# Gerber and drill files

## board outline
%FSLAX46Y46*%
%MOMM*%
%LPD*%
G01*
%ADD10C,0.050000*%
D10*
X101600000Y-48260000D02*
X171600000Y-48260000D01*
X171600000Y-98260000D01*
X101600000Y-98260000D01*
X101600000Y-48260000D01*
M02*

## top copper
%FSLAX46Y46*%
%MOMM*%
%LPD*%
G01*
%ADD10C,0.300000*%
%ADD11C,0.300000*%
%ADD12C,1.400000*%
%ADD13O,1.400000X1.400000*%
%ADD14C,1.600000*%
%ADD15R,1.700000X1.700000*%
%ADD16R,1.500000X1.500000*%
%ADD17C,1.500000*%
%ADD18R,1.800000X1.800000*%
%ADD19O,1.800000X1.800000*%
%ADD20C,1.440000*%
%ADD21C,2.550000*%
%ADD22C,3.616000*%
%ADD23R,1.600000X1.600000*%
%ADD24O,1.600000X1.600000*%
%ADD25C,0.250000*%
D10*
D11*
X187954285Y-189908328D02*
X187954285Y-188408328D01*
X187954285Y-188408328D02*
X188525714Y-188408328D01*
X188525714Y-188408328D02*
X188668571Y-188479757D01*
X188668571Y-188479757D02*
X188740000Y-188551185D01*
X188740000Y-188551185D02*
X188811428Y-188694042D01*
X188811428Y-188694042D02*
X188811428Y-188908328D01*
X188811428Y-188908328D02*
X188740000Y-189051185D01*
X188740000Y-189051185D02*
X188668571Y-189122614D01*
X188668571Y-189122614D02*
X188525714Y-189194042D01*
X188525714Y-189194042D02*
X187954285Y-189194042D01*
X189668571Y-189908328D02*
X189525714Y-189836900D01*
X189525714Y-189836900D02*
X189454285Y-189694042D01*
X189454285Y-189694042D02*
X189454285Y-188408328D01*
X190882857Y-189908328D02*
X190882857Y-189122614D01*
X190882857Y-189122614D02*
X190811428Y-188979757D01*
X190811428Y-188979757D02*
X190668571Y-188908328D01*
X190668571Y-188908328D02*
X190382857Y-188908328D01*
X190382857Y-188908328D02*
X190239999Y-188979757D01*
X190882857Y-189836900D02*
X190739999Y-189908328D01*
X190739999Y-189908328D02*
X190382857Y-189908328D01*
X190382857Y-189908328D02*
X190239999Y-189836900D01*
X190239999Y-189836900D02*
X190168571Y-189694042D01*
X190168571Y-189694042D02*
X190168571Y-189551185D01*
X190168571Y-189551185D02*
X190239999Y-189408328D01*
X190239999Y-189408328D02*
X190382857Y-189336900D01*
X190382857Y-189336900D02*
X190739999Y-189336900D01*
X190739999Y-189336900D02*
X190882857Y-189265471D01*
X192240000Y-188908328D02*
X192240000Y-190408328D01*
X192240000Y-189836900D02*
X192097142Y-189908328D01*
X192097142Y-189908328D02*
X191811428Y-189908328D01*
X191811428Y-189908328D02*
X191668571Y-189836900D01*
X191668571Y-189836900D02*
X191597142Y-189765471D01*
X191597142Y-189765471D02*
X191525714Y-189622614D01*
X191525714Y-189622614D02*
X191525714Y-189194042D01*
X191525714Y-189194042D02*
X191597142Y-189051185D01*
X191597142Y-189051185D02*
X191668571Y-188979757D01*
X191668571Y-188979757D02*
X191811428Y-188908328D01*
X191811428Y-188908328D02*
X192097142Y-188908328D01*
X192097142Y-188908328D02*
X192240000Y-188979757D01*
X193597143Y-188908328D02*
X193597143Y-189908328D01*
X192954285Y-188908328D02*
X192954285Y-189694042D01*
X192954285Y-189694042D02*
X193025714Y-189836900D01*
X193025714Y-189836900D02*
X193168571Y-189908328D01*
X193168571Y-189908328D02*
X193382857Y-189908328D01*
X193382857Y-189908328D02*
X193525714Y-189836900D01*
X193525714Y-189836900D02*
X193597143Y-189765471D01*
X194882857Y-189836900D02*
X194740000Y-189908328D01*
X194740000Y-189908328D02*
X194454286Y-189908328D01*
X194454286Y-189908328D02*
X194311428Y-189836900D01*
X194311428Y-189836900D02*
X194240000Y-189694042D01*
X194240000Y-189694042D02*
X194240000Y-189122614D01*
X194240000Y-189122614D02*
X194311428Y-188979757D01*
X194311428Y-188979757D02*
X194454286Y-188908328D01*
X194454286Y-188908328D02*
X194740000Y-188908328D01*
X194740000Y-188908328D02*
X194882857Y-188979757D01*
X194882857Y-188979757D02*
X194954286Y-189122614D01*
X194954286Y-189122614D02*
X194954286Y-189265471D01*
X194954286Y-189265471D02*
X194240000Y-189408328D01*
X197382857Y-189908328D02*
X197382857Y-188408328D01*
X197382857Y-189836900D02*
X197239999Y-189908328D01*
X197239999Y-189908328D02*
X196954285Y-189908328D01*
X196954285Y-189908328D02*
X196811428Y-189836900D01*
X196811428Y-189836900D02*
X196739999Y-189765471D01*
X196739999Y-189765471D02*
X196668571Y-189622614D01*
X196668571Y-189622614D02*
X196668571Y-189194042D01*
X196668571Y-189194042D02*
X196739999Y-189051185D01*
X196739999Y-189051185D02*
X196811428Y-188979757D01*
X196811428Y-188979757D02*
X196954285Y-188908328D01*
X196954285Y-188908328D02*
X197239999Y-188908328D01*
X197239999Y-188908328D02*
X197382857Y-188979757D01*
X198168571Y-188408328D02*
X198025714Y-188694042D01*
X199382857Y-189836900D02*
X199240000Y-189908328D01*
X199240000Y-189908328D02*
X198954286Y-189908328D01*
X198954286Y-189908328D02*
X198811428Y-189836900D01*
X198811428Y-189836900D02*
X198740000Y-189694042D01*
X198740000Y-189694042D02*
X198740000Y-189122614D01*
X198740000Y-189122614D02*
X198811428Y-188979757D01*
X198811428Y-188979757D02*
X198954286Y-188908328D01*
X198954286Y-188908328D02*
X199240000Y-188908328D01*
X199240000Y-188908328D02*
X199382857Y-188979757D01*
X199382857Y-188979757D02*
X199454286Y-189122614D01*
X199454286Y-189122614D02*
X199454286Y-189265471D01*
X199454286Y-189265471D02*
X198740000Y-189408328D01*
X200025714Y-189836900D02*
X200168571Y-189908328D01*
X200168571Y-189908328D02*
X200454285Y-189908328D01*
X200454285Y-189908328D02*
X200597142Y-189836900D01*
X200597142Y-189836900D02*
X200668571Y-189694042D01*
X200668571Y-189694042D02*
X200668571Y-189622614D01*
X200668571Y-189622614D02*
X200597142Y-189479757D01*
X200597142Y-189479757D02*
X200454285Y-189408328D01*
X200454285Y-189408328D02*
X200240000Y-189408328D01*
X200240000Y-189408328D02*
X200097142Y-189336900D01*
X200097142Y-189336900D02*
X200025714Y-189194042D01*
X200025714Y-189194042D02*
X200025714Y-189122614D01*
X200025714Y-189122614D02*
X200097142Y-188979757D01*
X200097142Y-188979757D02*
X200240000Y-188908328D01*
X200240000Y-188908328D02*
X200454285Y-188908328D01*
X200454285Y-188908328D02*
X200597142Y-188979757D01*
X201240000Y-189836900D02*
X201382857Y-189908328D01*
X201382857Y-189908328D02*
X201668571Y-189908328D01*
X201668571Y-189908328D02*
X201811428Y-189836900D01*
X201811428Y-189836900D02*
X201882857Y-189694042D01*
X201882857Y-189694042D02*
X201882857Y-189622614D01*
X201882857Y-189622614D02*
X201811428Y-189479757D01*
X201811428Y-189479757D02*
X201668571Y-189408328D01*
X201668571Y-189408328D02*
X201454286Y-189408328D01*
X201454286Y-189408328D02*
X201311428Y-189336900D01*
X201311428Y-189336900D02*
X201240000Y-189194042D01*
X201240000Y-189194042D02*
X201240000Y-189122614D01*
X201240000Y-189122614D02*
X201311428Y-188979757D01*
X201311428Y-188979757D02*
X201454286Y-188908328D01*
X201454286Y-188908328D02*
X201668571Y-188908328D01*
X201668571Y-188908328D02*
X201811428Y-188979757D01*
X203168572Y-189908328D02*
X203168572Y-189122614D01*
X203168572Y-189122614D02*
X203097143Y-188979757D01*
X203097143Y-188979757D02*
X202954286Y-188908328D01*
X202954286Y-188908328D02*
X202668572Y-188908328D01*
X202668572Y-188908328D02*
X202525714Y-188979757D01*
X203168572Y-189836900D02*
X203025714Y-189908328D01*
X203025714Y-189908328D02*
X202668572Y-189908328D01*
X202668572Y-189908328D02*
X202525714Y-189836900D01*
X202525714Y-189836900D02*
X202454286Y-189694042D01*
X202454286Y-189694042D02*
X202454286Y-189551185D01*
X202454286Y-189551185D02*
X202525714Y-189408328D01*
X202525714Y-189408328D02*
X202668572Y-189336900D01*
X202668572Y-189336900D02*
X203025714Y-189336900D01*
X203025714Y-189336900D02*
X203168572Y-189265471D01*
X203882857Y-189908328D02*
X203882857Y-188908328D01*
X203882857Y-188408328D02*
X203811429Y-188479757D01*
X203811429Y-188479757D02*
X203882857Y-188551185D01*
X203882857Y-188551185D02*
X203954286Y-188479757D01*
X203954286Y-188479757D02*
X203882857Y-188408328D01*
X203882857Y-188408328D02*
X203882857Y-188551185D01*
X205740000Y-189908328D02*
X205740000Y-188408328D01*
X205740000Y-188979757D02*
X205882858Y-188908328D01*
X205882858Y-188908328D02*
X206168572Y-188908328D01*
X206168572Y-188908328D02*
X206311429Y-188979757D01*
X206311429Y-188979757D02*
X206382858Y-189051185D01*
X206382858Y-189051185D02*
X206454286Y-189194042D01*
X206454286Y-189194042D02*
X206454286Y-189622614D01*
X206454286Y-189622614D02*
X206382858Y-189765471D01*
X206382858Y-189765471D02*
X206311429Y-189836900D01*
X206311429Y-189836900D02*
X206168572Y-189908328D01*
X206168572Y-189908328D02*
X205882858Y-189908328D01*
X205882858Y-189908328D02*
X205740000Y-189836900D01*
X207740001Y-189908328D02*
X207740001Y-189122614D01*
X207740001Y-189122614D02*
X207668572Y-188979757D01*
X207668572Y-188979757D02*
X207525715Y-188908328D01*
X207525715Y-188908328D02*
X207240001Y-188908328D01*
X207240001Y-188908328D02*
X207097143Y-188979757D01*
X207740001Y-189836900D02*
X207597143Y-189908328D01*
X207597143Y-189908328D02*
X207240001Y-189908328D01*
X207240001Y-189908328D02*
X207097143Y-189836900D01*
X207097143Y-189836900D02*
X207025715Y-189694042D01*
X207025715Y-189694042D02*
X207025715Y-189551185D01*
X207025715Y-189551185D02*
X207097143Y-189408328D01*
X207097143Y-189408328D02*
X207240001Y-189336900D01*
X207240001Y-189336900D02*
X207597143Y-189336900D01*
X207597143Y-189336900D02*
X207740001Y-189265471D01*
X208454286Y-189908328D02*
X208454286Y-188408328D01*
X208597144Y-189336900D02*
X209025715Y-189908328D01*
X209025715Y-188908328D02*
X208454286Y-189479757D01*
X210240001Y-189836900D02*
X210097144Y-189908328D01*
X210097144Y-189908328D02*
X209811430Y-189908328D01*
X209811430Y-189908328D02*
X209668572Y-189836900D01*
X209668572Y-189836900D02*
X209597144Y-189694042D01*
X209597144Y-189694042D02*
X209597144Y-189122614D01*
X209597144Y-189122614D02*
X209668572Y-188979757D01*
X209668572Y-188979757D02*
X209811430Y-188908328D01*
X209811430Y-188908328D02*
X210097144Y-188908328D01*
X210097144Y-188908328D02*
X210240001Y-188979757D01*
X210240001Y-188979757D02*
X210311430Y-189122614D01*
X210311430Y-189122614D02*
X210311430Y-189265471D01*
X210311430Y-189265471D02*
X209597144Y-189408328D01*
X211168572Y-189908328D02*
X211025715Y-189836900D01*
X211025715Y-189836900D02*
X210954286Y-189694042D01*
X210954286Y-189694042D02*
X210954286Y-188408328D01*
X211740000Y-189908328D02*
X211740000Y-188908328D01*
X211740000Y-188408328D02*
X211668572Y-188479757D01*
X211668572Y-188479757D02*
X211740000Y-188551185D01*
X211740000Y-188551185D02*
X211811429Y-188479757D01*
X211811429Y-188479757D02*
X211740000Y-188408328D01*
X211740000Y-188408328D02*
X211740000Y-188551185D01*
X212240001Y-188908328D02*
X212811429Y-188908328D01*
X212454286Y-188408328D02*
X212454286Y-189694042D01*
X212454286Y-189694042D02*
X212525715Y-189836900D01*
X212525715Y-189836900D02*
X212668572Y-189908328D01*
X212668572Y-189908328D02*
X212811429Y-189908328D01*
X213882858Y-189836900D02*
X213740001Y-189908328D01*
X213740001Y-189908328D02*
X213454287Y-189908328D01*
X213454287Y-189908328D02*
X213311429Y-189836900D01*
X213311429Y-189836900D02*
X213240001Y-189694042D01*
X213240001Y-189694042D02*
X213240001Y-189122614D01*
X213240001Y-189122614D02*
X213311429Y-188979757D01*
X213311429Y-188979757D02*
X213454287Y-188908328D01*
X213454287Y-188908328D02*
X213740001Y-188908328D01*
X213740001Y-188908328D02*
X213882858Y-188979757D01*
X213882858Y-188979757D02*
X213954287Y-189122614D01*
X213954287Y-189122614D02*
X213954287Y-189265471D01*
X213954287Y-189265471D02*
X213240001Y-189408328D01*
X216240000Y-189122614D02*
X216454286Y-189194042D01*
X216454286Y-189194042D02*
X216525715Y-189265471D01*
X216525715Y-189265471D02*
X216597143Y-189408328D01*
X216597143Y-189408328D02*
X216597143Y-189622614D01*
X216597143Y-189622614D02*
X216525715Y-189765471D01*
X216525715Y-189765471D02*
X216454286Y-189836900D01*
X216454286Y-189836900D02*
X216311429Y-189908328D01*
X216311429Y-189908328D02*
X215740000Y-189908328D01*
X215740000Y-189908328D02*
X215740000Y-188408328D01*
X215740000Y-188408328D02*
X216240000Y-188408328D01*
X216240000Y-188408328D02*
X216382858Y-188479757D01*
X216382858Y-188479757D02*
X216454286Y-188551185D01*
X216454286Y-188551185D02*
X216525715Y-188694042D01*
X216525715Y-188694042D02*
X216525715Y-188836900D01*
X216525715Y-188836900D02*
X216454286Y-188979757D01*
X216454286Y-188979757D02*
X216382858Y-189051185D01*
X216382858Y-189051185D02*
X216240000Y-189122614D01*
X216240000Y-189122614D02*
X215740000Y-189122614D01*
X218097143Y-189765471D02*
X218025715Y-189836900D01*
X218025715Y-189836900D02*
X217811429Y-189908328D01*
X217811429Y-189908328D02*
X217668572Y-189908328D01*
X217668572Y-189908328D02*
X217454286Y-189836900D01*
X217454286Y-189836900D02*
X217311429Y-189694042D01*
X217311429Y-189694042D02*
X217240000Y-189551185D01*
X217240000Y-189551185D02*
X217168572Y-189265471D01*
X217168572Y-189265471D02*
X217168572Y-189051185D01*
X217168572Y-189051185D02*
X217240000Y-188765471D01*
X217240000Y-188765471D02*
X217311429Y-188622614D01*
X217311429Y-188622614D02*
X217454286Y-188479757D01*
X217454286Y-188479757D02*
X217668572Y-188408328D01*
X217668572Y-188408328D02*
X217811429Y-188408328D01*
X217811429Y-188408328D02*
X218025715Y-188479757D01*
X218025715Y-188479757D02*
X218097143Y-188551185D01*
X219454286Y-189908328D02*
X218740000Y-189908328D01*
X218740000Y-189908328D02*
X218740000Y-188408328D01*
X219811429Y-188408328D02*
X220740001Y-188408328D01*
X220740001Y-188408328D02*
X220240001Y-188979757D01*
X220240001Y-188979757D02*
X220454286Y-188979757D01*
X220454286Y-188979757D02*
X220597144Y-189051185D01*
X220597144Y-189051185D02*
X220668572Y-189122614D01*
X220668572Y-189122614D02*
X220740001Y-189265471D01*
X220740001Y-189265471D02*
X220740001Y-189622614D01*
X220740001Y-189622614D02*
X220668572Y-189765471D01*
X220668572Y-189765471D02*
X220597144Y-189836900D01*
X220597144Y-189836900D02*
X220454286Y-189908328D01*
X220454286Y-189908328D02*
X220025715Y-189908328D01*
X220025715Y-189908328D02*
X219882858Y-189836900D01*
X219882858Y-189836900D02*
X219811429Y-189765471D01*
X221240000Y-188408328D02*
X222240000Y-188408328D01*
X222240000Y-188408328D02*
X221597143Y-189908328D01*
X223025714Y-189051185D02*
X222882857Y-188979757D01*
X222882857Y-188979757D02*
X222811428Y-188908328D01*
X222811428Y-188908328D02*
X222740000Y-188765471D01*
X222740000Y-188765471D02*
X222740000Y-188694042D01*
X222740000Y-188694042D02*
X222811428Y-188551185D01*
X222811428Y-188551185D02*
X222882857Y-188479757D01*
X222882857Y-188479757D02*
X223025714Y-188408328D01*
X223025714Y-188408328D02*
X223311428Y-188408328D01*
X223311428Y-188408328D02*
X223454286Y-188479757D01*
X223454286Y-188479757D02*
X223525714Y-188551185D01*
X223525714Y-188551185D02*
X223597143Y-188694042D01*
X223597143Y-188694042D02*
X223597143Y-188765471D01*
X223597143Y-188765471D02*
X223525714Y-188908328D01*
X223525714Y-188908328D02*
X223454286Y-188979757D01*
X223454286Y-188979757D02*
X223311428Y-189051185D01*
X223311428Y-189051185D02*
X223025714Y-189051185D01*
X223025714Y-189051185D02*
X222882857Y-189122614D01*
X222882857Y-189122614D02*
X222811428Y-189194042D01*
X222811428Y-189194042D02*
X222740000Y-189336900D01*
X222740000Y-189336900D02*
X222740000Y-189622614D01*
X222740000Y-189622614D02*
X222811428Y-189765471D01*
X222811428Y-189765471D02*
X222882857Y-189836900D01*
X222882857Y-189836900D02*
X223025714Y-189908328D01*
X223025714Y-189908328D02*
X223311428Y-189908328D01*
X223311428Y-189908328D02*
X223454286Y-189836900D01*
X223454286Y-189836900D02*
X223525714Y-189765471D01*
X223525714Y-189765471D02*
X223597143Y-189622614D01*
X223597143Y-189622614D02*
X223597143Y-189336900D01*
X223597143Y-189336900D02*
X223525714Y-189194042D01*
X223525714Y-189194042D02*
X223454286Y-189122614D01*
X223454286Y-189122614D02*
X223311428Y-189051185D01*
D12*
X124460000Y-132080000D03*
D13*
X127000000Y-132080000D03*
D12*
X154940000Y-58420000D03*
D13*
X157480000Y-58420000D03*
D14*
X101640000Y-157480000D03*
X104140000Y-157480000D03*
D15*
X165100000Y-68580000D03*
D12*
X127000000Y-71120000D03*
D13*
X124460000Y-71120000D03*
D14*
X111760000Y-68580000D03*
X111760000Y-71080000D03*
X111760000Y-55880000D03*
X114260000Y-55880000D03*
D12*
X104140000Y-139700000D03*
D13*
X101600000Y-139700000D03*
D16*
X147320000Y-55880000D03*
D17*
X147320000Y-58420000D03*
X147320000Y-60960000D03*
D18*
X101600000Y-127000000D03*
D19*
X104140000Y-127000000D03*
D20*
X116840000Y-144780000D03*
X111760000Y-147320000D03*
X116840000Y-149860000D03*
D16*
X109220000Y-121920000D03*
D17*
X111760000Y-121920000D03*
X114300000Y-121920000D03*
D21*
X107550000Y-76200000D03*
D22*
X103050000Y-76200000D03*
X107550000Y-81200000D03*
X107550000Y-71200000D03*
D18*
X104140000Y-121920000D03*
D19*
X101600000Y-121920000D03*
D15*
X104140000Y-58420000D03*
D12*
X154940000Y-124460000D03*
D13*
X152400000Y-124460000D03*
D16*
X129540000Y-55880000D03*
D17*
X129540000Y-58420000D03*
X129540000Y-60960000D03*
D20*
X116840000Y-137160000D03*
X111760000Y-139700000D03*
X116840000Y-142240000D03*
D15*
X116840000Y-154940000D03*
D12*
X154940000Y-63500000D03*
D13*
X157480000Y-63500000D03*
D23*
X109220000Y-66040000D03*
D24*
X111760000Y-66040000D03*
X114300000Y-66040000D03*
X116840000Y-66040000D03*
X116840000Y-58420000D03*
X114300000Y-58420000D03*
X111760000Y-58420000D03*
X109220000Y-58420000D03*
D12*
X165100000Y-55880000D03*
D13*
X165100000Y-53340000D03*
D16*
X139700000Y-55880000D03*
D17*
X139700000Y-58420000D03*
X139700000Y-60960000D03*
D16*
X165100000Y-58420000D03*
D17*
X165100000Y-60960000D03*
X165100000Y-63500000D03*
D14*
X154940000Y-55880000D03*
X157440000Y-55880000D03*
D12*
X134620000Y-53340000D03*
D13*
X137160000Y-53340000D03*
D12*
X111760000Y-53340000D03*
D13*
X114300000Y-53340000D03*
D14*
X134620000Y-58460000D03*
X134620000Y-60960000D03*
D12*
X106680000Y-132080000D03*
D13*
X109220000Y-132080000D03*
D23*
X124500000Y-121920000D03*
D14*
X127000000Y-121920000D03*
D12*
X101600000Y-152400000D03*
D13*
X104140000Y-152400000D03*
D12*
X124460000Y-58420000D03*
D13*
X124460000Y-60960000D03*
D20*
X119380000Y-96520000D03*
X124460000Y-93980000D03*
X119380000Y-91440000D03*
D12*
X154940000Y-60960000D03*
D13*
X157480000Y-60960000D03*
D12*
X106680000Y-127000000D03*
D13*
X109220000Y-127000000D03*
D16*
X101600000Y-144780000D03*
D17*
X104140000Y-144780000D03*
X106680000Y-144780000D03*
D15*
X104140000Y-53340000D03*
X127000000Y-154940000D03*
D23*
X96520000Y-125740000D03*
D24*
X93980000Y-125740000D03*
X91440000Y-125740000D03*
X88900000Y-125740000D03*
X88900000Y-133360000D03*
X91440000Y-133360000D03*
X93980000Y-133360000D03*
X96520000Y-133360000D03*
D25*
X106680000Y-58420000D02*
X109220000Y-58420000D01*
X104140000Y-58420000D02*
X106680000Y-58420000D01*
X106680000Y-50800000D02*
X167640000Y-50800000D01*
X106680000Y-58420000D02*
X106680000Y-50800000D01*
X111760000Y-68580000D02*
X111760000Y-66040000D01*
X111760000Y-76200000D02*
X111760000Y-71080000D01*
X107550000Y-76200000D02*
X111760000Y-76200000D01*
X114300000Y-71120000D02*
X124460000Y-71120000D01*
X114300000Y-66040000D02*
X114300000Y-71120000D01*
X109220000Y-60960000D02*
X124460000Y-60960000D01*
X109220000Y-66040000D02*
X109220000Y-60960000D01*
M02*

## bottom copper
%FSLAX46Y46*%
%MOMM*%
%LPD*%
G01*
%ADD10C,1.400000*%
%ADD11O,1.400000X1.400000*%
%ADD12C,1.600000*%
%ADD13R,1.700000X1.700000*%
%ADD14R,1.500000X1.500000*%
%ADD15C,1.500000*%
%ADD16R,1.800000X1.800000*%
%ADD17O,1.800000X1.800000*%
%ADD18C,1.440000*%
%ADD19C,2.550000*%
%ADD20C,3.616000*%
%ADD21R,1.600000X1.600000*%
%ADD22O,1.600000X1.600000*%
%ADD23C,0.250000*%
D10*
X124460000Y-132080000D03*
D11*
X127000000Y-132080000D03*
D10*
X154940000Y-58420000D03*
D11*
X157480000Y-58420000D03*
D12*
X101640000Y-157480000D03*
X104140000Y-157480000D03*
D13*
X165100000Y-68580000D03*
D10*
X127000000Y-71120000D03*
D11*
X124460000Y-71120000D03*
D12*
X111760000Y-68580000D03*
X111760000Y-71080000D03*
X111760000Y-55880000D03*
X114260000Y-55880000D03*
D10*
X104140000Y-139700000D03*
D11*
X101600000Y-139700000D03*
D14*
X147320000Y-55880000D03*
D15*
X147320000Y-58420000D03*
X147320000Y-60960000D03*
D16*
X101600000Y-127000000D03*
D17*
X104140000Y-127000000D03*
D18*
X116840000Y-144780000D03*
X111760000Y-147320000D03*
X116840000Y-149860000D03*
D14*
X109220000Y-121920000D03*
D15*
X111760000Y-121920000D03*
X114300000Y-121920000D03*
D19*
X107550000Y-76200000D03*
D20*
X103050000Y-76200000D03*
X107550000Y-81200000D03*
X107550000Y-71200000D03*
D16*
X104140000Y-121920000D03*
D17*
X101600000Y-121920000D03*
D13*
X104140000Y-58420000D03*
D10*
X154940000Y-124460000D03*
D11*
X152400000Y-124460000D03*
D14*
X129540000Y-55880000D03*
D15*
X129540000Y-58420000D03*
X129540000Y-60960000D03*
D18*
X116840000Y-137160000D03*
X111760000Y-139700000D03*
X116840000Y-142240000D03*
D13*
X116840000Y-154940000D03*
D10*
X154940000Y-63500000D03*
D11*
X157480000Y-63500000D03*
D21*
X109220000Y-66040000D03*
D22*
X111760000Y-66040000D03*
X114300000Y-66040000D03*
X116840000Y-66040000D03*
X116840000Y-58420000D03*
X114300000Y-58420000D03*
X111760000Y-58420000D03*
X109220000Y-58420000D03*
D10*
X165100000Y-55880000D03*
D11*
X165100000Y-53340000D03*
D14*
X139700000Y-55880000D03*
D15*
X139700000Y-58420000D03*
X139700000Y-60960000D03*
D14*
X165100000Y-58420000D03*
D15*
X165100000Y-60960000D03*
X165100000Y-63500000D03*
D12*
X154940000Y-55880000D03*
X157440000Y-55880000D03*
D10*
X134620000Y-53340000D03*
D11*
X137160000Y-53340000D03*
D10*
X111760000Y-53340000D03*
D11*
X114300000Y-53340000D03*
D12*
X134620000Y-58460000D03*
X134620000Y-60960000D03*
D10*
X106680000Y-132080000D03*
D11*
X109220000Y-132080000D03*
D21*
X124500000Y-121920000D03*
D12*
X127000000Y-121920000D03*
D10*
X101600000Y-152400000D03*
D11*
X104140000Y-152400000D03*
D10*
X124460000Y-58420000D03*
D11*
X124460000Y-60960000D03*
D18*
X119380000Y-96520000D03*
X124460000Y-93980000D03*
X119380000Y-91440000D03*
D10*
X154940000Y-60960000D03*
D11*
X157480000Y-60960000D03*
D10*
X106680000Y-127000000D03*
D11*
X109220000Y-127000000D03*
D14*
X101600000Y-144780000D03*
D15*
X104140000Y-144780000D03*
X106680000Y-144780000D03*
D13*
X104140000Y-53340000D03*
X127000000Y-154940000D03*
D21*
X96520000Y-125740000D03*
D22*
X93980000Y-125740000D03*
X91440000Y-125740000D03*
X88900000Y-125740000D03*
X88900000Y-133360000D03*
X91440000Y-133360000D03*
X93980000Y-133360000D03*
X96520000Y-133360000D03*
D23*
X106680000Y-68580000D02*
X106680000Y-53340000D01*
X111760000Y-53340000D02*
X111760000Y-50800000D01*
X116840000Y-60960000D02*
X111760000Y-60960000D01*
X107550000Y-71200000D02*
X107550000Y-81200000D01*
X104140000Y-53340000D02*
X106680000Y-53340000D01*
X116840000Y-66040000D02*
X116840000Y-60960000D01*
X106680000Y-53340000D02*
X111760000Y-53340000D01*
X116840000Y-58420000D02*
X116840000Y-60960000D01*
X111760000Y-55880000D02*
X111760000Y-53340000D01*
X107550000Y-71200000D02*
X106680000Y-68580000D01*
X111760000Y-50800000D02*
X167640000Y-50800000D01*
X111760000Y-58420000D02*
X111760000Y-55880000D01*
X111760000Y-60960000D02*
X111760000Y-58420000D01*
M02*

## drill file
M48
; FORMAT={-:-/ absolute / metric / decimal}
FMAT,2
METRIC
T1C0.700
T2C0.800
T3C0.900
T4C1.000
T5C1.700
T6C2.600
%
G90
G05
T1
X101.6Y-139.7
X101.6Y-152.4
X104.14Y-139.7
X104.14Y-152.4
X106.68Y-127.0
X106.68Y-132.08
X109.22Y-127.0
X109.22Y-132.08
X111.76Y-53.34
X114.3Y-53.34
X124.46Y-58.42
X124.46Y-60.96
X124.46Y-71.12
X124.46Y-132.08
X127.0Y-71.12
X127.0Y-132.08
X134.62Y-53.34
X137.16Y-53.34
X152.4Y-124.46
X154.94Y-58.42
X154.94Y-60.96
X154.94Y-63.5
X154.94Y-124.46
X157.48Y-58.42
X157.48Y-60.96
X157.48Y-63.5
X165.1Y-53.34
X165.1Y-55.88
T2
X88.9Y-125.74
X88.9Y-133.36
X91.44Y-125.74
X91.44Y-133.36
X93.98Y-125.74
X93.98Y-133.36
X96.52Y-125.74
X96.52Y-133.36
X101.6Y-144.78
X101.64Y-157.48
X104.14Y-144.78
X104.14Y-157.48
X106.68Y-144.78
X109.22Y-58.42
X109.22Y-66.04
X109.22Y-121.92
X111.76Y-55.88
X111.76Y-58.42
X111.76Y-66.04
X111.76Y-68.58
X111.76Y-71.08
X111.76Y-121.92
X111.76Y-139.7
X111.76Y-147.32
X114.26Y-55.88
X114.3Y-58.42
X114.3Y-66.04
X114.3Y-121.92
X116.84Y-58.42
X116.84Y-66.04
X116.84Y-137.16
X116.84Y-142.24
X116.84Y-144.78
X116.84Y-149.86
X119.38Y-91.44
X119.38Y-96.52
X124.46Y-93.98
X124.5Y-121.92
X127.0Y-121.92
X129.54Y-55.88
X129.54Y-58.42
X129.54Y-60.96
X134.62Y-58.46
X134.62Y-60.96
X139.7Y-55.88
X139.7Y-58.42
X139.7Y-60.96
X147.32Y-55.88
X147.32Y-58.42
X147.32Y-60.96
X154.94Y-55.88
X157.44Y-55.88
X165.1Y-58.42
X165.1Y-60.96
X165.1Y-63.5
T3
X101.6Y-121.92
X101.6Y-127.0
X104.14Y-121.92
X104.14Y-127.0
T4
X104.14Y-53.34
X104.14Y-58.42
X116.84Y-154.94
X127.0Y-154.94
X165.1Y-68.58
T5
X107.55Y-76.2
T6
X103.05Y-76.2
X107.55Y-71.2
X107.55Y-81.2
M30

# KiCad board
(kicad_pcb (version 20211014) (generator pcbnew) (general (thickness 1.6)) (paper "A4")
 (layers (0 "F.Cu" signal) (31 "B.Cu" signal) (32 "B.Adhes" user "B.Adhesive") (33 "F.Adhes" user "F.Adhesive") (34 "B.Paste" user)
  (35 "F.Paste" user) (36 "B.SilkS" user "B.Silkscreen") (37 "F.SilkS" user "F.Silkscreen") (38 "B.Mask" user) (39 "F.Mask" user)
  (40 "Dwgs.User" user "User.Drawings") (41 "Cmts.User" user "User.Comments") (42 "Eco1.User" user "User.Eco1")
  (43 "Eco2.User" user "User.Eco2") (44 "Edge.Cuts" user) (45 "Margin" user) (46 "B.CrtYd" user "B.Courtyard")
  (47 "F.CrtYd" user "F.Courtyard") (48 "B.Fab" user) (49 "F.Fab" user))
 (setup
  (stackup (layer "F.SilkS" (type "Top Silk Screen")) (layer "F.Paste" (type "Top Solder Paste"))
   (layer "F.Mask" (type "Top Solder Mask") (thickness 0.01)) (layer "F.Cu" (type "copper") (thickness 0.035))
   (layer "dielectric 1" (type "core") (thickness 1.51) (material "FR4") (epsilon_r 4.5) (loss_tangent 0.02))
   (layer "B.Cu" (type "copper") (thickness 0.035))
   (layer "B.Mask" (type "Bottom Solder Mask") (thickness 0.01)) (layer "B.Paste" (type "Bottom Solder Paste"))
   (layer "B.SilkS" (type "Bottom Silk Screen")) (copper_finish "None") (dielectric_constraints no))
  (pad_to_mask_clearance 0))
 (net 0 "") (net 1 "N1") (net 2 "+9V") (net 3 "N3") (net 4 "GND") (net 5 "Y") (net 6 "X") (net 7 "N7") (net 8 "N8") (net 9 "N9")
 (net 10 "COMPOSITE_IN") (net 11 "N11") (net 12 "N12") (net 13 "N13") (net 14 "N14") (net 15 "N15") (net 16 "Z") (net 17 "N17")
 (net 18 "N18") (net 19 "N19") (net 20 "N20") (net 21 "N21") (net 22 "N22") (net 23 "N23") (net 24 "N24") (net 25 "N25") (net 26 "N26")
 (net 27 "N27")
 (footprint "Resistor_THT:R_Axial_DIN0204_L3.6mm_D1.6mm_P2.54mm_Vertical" (layer "F.Cu") (at 124.46 132.08)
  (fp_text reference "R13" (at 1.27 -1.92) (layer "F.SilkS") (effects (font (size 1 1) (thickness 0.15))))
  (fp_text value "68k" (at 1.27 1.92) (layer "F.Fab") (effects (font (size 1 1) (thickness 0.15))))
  (pad "1" thru_hole circle (at 0 0) (size 1.4 1.4) (drill 0.7) (layers *.Cu *.Mask) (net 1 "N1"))
  (pad "2" thru_hole oval (at 2.54 0) (size 1.4 1.4) (drill 0.7) (layers *.Cu *.Mask) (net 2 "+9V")))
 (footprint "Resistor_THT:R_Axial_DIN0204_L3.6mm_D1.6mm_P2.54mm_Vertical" (layer "F.Cu") (at 154.94 58.42)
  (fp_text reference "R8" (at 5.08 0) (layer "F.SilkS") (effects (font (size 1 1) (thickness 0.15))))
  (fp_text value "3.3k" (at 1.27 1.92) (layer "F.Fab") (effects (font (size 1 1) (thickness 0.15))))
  (pad "1" thru_hole circle (at 0 0) (size 1.4 1.4) (drill 0.7) (layers *.Cu *.Mask) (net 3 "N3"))
  (pad "2" thru_hole oval (at 2.54 0) (size 1.4 1.4) (drill 0.7) (layers *.Cu *.Mask) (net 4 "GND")))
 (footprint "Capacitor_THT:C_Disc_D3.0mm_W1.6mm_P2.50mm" (layer "F.Cu") (at 101.64 157.48)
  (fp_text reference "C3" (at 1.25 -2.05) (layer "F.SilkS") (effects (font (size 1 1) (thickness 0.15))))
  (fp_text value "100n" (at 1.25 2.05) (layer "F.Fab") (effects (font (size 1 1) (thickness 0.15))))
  (pad "1" thru_hole circle (at 0 0) (size 1.6 1.6) (drill 0.8) (layers *.Cu *.Mask) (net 2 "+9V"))
  (pad "2" thru_hole circle (at 2.5 0) (size 1.6 1.6) (drill 0.8) (layers *.Cu *.Mask) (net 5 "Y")))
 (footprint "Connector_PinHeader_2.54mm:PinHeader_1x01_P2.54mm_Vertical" (layer "F.Cu") (at 165.1 68.58)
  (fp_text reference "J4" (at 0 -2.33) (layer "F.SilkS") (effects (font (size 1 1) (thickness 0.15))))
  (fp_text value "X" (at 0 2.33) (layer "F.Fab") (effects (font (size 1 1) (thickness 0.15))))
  (pad "1" thru_hole rect (at 0 0) (size 1.7 1.7) (drill 1) (layers *.Cu *.Mask) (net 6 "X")))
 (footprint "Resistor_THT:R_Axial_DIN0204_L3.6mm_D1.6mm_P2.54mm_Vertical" (layer "F.Cu") (at 127 71.12 180)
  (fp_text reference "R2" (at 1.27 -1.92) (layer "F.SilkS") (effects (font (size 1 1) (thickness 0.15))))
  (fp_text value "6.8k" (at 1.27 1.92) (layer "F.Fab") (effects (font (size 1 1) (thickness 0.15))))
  (pad "1" thru_hole circle (at 0 0 180) (size 1.4 1.4) (drill 0.7) (layers *.Cu *.Mask) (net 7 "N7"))
  (pad "2" thru_hole oval (at 2.54 0 180) (size 1.4 1.4) (drill 0.7) (layers *.Cu *.Mask) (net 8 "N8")))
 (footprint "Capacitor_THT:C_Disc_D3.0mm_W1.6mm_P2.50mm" (layer "F.Cu") (at 111.76 68.58 -90)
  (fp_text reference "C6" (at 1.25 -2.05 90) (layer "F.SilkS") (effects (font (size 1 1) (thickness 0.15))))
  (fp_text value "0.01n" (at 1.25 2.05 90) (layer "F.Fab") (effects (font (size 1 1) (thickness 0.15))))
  (pad "1" thru_hole circle (at 0 0 270) (size 1.6 1.6) (drill 0.8) (layers *.Cu *.Mask) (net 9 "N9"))
  (pad "2" thru_hole circle (at 2.5 0 270) (size 1.6 1.6) (drill 0.8) (layers *.Cu *.Mask) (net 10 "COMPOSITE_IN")))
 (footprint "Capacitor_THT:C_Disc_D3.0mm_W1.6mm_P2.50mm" (layer "F.Cu") (at 111.76 55.88)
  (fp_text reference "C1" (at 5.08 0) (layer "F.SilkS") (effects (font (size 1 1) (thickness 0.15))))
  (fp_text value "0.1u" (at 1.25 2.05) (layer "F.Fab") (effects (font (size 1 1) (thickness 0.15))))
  (pad "1" thru_hole circle (at 0 0) (size 1.6 1.6) (drill 0.8) (layers *.Cu *.Mask) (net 4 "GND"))
  (pad "2" thru_hole circle (at 2.5 0) (size 1.6 1.6) (drill 0.8) (layers *.Cu *.Mask) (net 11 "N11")))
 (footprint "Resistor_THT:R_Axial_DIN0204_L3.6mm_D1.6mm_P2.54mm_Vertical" (layer "F.Cu") (at 104.14 139.7 180)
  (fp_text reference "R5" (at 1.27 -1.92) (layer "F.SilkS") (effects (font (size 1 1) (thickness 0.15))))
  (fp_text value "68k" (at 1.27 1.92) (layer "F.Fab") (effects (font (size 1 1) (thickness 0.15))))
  (pad "1" thru_hole circle (at 0 0 180) (size 1.4 1.4) (drill 0.7) (layers *.Cu *.Mask) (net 4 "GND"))
  (pad "2" thru_hole oval (at 2.54 0 180) (size 1.4 1.4) (drill 0.7) (layers *.Cu *.Mask) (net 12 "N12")))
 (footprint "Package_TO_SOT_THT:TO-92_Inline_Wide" (layer "F.Cu") (at 147.32 55.88 -90)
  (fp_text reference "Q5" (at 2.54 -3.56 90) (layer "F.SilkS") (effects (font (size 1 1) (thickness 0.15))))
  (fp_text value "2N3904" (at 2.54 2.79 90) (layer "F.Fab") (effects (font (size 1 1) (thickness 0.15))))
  (pad "1" thru_hole rect (at 0 0 270) (size 1.5 1.5) (drill 0.8) (layers *.Cu *.Mask) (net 3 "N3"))
  (pad "2" thru_hole circle (at 2.54 0 270) (size 1.5 1.5) (drill 0.8) (layers *.Cu *.Mask) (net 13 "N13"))
  (pad "3" thru_hole circle (at 5.08 0 270) (size 1.5 1.5) (drill 0.8) (layers *.Cu *.Mask) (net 2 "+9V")))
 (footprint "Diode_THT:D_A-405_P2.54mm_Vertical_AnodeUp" (layer "F.Cu") (at 101.6 127)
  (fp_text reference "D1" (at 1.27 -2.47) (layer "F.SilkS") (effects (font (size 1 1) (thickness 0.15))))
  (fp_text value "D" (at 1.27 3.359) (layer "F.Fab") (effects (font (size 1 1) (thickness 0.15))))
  (pad "1" thru_hole rect (at 0 0) (size 1.8 1.8) (drill 0.9) (layers *.Cu *.Mask) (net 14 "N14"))
  (pad "2" thru_hole oval (at 2.54 0) (size 1.8 1.8) (drill 0.9) (layers *.Cu *.Mask) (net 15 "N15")))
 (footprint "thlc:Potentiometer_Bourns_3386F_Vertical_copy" (layer "F.Cu") (at 116.84 144.78 180)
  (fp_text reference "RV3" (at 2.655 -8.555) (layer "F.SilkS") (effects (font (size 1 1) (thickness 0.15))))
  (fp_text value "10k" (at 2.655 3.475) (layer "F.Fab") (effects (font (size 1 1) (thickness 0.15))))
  (pad "1" thru_hole circle (at 0 0 180) (size 1.44 1.44) (drill 0.8) (layers *.Cu *.Mask) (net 4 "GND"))
  (pad "2" thru_hole circle (at 5.08 -2.54 180) (size 1.44 1.44) (drill 0.8) (layers *.Cu *.Mask) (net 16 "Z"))
  (pad "3" thru_hole circle (at 0 -5.08 180) (size 1.44 1.44) (drill 0.8) (layers *.Cu *.Mask) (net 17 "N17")))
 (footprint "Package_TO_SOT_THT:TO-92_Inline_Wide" (layer "F.Cu") (at 109.22 121.92)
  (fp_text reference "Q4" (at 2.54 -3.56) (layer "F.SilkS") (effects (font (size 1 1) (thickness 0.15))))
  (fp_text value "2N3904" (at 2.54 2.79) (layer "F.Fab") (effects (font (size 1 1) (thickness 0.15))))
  (pad "1" thru_hole rect (at 0 0) (size 1.5 1.5) (drill 0.8) (layers *.Cu *.Mask) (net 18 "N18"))
  (pad "2" thru_hole circle (at 2.54 0) (size 1.5 1.5) (drill 0.8) (layers *.Cu *.Mask) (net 15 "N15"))
  (pad "3" thru_hole circle (at 5.08 0) (size 1.5 1.5) (drill 0.8) (layers *.Cu *.Mask) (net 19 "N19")))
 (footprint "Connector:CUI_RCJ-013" (layer "F.Cu") (at 101.6 76.2)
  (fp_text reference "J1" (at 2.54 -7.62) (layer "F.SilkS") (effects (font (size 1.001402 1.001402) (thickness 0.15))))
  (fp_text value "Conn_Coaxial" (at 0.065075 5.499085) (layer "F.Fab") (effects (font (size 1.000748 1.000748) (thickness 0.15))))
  (pad "1" thru_hole circle (at 5.95 0) (size 2.55 2.55) (drill 1.7) (layers *.Cu *.Mask) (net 10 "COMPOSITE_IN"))
  (pad "2" thru_hole circle (at 1.45 0) (size 3.616 3.616) (drill 2.6) (layers *.Cu *.Mask) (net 4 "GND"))
  (pad "2" thru_hole circle (at 5.95 5) (size 3.616 3.616) (drill 2.6) (layers *.Cu *.Mask) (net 4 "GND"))
  (pad "2" thru_hole circle (at 5.95 -5) (size 3.616 3.616) (drill 2.6) (layers *.Cu *.Mask) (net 4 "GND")))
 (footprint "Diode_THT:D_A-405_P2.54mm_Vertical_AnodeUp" (layer "F.Cu") (at 104.14 121.92 180)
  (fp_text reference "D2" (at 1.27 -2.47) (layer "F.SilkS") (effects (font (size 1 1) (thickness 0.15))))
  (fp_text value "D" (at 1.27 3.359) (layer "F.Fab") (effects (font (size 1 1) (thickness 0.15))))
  (pad "1" thru_hole rect (at 0 0 180) (size 1.8 1.8) (drill 0.9) (layers *.Cu *.Mask) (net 4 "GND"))
  (pad "2" thru_hole oval (at 2.54 0 180) (size 1.8 1.8) (drill 0.9) (layers *.Cu *.Mask) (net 14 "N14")))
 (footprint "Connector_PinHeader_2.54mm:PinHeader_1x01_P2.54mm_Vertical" (layer "F.Cu") (at 104.14 58.42)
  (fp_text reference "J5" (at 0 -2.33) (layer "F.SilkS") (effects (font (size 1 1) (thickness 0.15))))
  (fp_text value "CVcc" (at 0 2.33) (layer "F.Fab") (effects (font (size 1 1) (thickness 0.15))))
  (pad "1" thru_hole rect (at 0 0) (size 1.7 1.7) (drill 1) (layers *.Cu *.Mask) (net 2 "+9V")))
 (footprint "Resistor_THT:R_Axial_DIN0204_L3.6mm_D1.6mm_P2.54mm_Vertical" (layer "F.Cu") (at 154.94 124.46 180)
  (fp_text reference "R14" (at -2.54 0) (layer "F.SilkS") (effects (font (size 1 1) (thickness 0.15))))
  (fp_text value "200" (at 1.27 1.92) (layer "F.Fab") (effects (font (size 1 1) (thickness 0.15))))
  (pad "1" thru_hole circle (at 0 0 180) (size 1.4 1.4) (drill 0.7) (layers *.Cu *.Mask) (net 16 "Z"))
  (pad "2" thru_hole oval (at 2.54 0 180) (size 1.4 1.4) (drill 0.7) (layers *.Cu *.Mask) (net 4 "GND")))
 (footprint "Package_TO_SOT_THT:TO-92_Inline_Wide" (layer "F.Cu") (at 129.54 55.88 -90)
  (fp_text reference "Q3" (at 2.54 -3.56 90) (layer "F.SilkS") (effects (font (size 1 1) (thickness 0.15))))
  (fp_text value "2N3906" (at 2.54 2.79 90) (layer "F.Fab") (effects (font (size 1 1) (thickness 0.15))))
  (pad "1" thru_hole rect (at 0 0 270) (size 1.5 1.5) (drill 0.8) (layers *.Cu *.Mask) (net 2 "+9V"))
  (pad "2" thru_hole circle (at 2.54 0 270) (size 1.5 1.5) (drill 0.8) (layers *.Cu *.Mask) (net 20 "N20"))
  (pad "3" thru_hole circle (at 5.08 0 270) (size 1.5 1.5) (drill 0.8) (layers *.Cu *.Mask) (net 19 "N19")))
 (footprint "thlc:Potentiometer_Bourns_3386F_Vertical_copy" (layer "F.Cu") (at 116.84 137.16 180)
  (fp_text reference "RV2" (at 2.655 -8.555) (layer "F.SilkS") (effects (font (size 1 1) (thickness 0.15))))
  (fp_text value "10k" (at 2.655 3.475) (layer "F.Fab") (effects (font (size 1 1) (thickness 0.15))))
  (pad "1" thru_hole circle (at 0 0 180) (size 1.44 1.44) (drill 0.8) (layers *.Cu *.Mask) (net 1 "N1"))
  (pad "2" thru_hole circle (at 5.08 -2.54 180) (size 1.44 1.44) (drill 0.8) (layers *.Cu *.Mask) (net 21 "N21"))
  (pad "3" thru_hole circle (at 0 -5.08 180) (size 1.44 1.44) (drill 0.8) (layers *.Cu *.Mask) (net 4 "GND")))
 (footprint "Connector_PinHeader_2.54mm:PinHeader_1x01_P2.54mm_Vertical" (layer "F.Cu") (at 116.84 154.94)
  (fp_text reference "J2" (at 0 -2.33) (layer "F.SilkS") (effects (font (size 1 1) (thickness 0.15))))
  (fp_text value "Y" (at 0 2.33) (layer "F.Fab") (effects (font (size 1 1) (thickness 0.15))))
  (pad "1" thru_hole rect (at 0 0) (size 1.7 1.7) (drill 1) (layers *.Cu *.Mask) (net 5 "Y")))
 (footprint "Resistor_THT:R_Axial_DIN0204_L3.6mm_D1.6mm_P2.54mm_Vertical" (layer "F.Cu") (at 154.94 63.5)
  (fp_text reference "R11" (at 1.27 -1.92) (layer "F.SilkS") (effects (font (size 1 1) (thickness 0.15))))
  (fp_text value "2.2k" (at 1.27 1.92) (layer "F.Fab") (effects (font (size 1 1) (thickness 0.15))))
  (pad "1" thru_hole circle (at 0 0) (size 1.4 1.4) (drill 0.7) (layers *.Cu *.Mask) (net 2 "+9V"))
  (pad "2" thru_hole oval (at 2.54 0) (size 1.4 1.4) (drill 0.7) (layers *.Cu *.Mask) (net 6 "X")))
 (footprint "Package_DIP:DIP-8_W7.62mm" (layer "F.Cu") (at 109.22 66.04 90)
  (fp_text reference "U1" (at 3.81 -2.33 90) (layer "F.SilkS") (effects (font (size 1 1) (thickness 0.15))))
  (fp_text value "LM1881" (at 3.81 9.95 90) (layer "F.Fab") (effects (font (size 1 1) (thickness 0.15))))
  (pad "1" thru_hole rect (at 0 0 90) (size 1.6 1.6) (drill 0.8) (layers *.Cu *.Mask) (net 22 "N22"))
  (pad "2" thru_hole oval (at 0 2.54 90) (size 1.6 1.6) (drill 0.8) (layers *.Cu *.Mask) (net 9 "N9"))
  (pad "3" thru_hole oval (at 0 5.08 90) (size 1.6 1.6) (drill 0.8) (layers *.Cu *.Mask) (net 8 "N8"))
  (pad "4" thru_hole oval (at 0 7.62 90) (size 1.6 1.6) (drill 0.8) (layers *.Cu *.Mask) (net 4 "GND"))
  (pad "5" thru_hole oval (at 7.62 7.62 90) (size 1.6 1.6) (drill 0.8) (layers *.Cu *.Mask) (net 4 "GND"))
  (pad "6" thru_hole oval (at 7.62 5.08 90) (size 1.6 1.6) (drill 0.8) (layers *.Cu *.Mask) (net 11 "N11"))
  (pad "7" thru_hole oval (at 7.62 2.54 90) (size 1.6 1.6) (drill 0.8) (layers *.Cu *.Mask) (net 4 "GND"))
  (pad "8" thru_hole oval (at 7.62 0 90) (size 1.6 1.6) (drill 0.8) (layers *.Cu *.Mask) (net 2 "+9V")))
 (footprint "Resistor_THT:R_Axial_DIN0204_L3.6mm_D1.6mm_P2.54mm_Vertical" (layer "F.Cu") (at 165.1 55.88 90)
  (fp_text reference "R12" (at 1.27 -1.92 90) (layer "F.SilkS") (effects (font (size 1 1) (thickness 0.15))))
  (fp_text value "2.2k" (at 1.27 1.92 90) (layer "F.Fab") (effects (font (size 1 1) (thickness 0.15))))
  (pad "1" thru_hole circle (at 0 0 90) (size 1.4 1.4) (drill 0.7) (layers *.Cu *.Mask) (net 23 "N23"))
  (pad "2" thru_hole oval (at 2.54 0 90) (size 1.4 1.4) (drill 0.7) (layers *.Cu *.Mask) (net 4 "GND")))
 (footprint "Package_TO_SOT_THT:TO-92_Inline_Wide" (layer "F.Cu") (at 139.7 55.88 -90)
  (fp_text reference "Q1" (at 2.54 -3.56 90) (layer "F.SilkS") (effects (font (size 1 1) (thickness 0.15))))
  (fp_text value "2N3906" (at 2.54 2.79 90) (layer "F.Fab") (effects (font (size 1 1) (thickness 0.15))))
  (pad "1" thru_hole rect (at 0 0 270) (size 1.5 1.5) (drill 0.8) (layers *.Cu *.Mask) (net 2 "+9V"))
  (pad "2" thru_hole circle (at 2.54 0 270) (size 1.5 1.5) (drill 0.8) (layers *.Cu *.Mask) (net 7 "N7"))
  (pad "3" thru_hole circle (at 5.08 0 270) (size 1.5 1.5) (drill 0.8) (layers *.Cu *.Mask) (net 5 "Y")))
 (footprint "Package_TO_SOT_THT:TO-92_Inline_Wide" (layer "F.Cu") (at 165.1 58.42 -90)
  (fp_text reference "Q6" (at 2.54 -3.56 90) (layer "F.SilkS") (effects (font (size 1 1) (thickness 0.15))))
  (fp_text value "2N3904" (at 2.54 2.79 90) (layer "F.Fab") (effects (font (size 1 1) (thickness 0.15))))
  (pad "1" thru_hole rect (at 0 0 270) (size 1.5 1.5) (drill 0.8) (layers *.Cu *.Mask) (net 23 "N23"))
  (pad "2" thru_hole circle (at 2.54 0 270) (size 1.5 1.5) (drill 0.8) (layers *.Cu *.Mask) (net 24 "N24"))
  (pad "3" thru_hole circle (at 5.08 0 270) (size 1.5 1.5) (drill 0.8) (layers *.Cu *.Mask) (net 6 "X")))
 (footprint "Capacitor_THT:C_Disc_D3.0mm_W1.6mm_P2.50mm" (layer "F.Cu") (at 154.94 55.88)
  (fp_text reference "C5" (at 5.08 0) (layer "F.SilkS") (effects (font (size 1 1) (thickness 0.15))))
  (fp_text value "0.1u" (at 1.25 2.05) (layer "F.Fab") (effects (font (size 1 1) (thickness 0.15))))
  (pad "1" thru_hole circle (at 0 0) (size 1.6 1.6) (drill 0.8) (layers *.Cu *.Mask) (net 3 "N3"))
  (pad "2" thru_hole circle (at 2.5 0) (size 1.6 1.6) (drill 0.8) (layers *.Cu *.Mask) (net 24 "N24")))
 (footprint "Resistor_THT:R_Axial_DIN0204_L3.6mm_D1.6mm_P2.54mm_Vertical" (layer "F.Cu") (at 134.62 53.34)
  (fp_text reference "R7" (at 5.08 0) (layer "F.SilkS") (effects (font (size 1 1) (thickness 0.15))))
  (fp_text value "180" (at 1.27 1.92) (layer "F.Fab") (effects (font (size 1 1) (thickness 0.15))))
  (pad "1" thru_hole circle (at 0 0) (size 1.4 1.4) (drill 0.7) (layers *.Cu *.Mask) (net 19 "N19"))
  (pad "2" thru_hole oval (at 2.54 0) (size 1.4 1.4) (drill 0.7) (layers *.Cu *.Mask) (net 13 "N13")))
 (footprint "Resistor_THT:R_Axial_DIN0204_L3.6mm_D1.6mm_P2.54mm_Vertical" (layer "F.Cu") (at 111.76 53.34)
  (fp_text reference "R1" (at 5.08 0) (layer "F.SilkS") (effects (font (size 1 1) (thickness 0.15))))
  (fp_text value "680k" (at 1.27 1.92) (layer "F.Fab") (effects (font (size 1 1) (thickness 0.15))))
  (pad "1" thru_hole circle (at 0 0) (size 1.4 1.4) (drill 0.7) (layers *.Cu *.Mask) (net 4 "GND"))
  (pad "2" thru_hole oval (at 2.54 0) (size 1.4 1.4) (drill 0.7) (layers *.Cu *.Mask) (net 11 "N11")))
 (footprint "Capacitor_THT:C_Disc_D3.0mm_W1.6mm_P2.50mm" (layer "F.Cu") (at 134.62 58.46 -90)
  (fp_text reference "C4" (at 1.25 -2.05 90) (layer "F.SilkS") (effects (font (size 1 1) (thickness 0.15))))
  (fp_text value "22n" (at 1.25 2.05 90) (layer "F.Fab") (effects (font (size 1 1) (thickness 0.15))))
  (pad "1" thru_hole circle (at 0 0 270) (size 1.6 1.6) (drill 0.8) (layers *.Cu *.Mask) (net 2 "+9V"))
  (pad "2" thru_hole circle (at 2.5 0 270) (size 1.6 1.6) (drill 0.8) (layers *.Cu *.Mask) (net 19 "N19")))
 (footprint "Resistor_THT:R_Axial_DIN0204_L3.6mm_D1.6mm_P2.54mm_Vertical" (layer "F.Cu") (at 106.68 132.08)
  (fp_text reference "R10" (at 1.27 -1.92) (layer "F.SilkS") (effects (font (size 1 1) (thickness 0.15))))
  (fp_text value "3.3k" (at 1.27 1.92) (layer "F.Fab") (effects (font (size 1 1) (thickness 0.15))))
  (pad "1" thru_hole circle (at 0 0) (size 1.4 1.4) (drill 0.7) (layers *.Cu *.Mask) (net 24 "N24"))
  (pad "2" thru_hole oval (at 2.54 0) (size 1.4 1.4) (drill 0.7) (layers *.Cu *.Mask) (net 4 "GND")))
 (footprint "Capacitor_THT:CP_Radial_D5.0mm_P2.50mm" (layer "F.Cu") (at 124.5 121.92)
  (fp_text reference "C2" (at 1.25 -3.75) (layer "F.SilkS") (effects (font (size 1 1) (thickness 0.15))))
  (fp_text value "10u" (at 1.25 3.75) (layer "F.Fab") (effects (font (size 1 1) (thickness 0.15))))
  (pad "1" thru_hole rect (at 0 0) (size 1.6 1.6) (drill 0.8) (layers *.Cu *.Mask) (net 2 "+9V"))
  (pad "2" thru_hole circle (at 2.5 0) (size 1.6 1.6) (drill 0.8) (layers *.Cu *.Mask) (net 4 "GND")))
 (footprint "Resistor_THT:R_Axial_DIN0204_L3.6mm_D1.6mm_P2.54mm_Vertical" (layer "F.Cu") (at 101.6 152.4)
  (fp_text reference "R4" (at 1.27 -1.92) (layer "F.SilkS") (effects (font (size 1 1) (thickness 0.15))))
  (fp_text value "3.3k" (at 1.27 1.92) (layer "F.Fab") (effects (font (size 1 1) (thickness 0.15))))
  (pad "1" thru_hole circle (at 0 0) (size 1.4 1.4) (drill 0.7) (layers *.Cu *.Mask) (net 2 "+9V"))
  (pad "2" thru_hole oval (at 2.54 0) (size 1.4 1.4) (drill 0.7) (layers *.Cu *.Mask) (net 15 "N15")))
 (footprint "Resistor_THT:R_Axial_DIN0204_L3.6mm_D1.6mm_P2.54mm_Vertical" (layer "F.Cu") (at 124.46 58.42 -90)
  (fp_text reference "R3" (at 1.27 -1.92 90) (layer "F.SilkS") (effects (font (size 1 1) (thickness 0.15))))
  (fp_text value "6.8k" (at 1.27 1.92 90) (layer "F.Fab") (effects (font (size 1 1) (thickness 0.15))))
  (pad "1" thru_hole circle (at 0 0 270) (size 1.4 1.4) (drill 0.7) (layers *.Cu *.Mask) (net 20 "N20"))
  (pad "2" thru_hole oval (at 2.54 0 270) (size 1.4 1.4) (drill 0.7) (layers *.Cu *.Mask) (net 22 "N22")))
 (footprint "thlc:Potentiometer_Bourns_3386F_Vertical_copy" (layer "F.Cu") (at 119.38 96.52)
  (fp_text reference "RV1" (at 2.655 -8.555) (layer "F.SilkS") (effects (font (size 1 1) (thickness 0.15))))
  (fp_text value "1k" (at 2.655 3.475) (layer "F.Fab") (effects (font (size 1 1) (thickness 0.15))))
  (pad "1" thru_hole circle (at 0 0) (size 1.44 1.44) (drill 0.8) (layers *.Cu *.Mask) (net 10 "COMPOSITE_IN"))
  (pad "2" thru_hole circle (at 5.08 -2.54) (size 1.44 1.44) (drill 0.8) (layers *.Cu *.Mask) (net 17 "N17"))
  (pad "3" thru_hole circle (at 0 -5.08) (size 1.44 1.44) (drill 0.8) (layers *.Cu *.Mask) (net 4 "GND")))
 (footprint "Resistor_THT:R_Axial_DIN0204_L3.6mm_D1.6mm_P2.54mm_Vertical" (layer "F.Cu") (at 154.94 60.96)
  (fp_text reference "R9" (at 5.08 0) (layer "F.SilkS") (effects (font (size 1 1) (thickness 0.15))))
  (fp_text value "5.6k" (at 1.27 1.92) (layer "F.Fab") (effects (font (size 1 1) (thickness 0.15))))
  (pad "1" thru_hole circle (at 0 0) (size 1.4 1.4) (drill 0.7) (layers *.Cu *.Mask) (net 2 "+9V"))
  (pad "2" thru_hole oval (at 2.54 0) (size 1.4 1.4) (drill 0.7) (layers *.Cu *.Mask) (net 24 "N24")))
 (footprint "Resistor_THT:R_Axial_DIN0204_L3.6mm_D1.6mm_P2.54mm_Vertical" (layer "F.Cu") (at 106.68 127)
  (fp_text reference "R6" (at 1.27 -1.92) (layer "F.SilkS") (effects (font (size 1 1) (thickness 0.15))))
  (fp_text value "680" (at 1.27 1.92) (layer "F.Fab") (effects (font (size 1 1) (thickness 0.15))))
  (pad "1" thru_hole circle (at 0 0) (size 1.4 1.4) (drill 0.7) (layers *.Cu *.Mask) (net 4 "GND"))
  (pad "2" thru_hole oval (at 2.54 0) (size 1.4 1.4) (drill 0.7) (layers *.Cu *.Mask) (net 18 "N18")))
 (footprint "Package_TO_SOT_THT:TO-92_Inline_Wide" (layer "F.Cu") (at 101.6 144.78)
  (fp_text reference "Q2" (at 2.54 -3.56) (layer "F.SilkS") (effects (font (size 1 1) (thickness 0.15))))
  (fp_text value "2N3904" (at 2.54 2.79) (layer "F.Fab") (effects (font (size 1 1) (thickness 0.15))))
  (pad "1" thru_hole rect (at 0 0) (size 1.5 1.5) (drill 0.8) (layers *.Cu *.Mask) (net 12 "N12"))
  (pad "2" thru_hole circle (at 2.54 0) (size 1.5 1.5) (drill 0.8) (layers *.Cu *.Mask) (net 15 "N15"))
  (pad "3" thru_hole circle (at 5.08 0) (size 1.5 1.5) (drill 0.8) (layers *.Cu *.Mask) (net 5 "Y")))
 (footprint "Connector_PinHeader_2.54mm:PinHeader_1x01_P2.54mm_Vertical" (layer "F.Cu") (at 104.14 53.34)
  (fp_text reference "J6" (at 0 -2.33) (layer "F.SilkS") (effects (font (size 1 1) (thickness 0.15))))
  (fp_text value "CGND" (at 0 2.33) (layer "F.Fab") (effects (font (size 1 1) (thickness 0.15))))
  (pad "1" thru_hole rect (at 0 0) (size 1.7 1.7) (drill 1) (layers *.Cu *.Mask) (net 4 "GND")))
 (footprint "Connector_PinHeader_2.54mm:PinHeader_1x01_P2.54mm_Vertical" (layer "F.Cu") (at 127 154.94)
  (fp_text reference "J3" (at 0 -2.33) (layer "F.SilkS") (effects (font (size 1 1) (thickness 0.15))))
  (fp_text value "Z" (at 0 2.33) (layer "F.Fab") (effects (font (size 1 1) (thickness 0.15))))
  (pad "1" thru_hole rect (at 0 0) (size 1.7 1.7) (drill 1) (layers *.Cu *.Mask) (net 16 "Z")))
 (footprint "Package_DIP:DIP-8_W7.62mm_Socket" (layer "F.Cu") (at 96.52 125.74 -90)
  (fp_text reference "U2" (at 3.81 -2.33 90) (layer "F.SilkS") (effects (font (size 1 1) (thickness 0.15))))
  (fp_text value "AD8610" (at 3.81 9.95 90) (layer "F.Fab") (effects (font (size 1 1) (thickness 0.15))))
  (pad "1" thru_hole rect (at 0 0 270) (size 1.6 1.6) (drill 0.8) (layers *.Cu *.Mask) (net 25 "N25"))
  (pad "2" thru_hole oval (at 0 2.54 270) (size 1.6 1.6) (drill 0.8) (layers *.Cu *.Mask) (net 17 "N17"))
  (pad "3" thru_hole oval (at 0 5.08 270) (size 1.6 1.6) (drill 0.8) (layers *.Cu *.Mask) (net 21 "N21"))
  (pad "4" thru_hole oval (at 0 7.62 270) (size 1.6 1.6) (drill 0.8) (layers *.Cu *.Mask) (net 4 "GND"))
  (pad "5" thru_hole oval (at 7.62 7.62 270) (size 1.6 1.6) (drill 0.8) (layers *.Cu *.Mask) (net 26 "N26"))
  (pad "6" thru_hole oval (at 7.62 5.08 270) (size 1.6 1.6) (drill 0.8) (layers *.Cu *.Mask) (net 16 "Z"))
  (pad "7" thru_hole oval (at 7.62 2.54 270) (size 1.6 1.6) (drill 0.8) (layers *.Cu *.Mask) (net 2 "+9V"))
  (pad "8" thru_hole oval (at 7.62 0 270) (size 1.6 1.6) (drill 0.8) (layers *.Cu *.Mask) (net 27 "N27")))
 (gr_rect (start 101.6 48.26) (end 171.6 98.26) (layer "Edge.Cuts") (width 0.05) (fill none))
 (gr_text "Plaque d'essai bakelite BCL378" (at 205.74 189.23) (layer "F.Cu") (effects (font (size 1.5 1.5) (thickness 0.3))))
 (segment (start 106.68 68.58) (end 106.68 53.34) (width 0.25) (layer "B.Cu") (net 4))
 (segment (start 111.76 53.34) (end 111.76 50.8) (width 0.25) (layer "B.Cu") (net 4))
 (segment (start 116.84 60.96) (end 111.76 60.96) (width 0.25) (layer "B.Cu") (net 4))
 (segment (start 107.55 71.2) (end 107.55 81.2) (width 0.25) (layer "B.Cu") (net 4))
 (segment (start 104.14 53.34) (end 106.68 53.34) (width 0.25) (layer "B.Cu") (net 4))
 (segment (start 116.84 66.04) (end 116.84 60.96) (width 0.25) (layer "B.Cu") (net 4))
 (segment (start 106.68 53.34) (end 111.76 53.34) (width 0.25) (layer "B.Cu") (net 4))
 (segment (start 116.84 58.42) (end 116.84 60.96) (width 0.25) (layer "B.Cu") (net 4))
 (segment (start 111.76 55.88) (end 111.76 53.34) (width 0.25) (layer "B.Cu") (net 4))
 (segment (start 107.55 71.2) (end 106.68 68.58) (width 0.25) (layer "B.Cu") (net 4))
 (segment (start 111.76 50.8) (end 167.64 50.8) (width 0.25) (layer "B.Cu") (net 4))
 (segment (start 111.76 58.42) (end 111.76 55.88) (width 0.25) (layer "B.Cu") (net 4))
 (segment (start 111.76 60.96) (end 111.76 58.42) (width 0.25) (layer "B.Cu") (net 4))
 (segment (start 106.68 58.42) (end 109.22 58.42) (width 0.25) (layer "F.Cu") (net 2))
 (segment (start 104.14 58.42) (end 106.68 58.42) (width 0.25) (layer "F.Cu") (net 2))
 (segment (start 106.68 50.8) (end 167.64 50.8) (width 0.25) (layer "F.Cu") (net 2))
 (segment (start 106.68 58.42) (end 106.68 50.8) (width 0.25) (layer "F.Cu") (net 2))
 (segment (start 111.76 68.58) (end 111.76 66.04) (width 0.25) (layer "F.Cu") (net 9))
 (segment (start 111.76 76.2) (end 111.76 71.08) (width 0.25) (layer "F.Cu") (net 10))
 (segment (start 107.55 76.2) (end 111.76 76.2) (width 0.25) (layer "F.Cu") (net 10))
 (segment (start 114.3 71.12) (end 124.46 71.12) (width 0.25) (layer "F.Cu") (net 8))
 (segment (start 114.3 66.04) (end 114.3 71.12) (width 0.25) (layer "F.Cu") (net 8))
 (segment (start 109.22 60.96) (end 124.46 60.96) (width 0.25) (layer "F.Cu") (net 22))
 (segment (start 109.22 66.04) (end 109.22 60.96) (width 0.25) (layer "F.Cu") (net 22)))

